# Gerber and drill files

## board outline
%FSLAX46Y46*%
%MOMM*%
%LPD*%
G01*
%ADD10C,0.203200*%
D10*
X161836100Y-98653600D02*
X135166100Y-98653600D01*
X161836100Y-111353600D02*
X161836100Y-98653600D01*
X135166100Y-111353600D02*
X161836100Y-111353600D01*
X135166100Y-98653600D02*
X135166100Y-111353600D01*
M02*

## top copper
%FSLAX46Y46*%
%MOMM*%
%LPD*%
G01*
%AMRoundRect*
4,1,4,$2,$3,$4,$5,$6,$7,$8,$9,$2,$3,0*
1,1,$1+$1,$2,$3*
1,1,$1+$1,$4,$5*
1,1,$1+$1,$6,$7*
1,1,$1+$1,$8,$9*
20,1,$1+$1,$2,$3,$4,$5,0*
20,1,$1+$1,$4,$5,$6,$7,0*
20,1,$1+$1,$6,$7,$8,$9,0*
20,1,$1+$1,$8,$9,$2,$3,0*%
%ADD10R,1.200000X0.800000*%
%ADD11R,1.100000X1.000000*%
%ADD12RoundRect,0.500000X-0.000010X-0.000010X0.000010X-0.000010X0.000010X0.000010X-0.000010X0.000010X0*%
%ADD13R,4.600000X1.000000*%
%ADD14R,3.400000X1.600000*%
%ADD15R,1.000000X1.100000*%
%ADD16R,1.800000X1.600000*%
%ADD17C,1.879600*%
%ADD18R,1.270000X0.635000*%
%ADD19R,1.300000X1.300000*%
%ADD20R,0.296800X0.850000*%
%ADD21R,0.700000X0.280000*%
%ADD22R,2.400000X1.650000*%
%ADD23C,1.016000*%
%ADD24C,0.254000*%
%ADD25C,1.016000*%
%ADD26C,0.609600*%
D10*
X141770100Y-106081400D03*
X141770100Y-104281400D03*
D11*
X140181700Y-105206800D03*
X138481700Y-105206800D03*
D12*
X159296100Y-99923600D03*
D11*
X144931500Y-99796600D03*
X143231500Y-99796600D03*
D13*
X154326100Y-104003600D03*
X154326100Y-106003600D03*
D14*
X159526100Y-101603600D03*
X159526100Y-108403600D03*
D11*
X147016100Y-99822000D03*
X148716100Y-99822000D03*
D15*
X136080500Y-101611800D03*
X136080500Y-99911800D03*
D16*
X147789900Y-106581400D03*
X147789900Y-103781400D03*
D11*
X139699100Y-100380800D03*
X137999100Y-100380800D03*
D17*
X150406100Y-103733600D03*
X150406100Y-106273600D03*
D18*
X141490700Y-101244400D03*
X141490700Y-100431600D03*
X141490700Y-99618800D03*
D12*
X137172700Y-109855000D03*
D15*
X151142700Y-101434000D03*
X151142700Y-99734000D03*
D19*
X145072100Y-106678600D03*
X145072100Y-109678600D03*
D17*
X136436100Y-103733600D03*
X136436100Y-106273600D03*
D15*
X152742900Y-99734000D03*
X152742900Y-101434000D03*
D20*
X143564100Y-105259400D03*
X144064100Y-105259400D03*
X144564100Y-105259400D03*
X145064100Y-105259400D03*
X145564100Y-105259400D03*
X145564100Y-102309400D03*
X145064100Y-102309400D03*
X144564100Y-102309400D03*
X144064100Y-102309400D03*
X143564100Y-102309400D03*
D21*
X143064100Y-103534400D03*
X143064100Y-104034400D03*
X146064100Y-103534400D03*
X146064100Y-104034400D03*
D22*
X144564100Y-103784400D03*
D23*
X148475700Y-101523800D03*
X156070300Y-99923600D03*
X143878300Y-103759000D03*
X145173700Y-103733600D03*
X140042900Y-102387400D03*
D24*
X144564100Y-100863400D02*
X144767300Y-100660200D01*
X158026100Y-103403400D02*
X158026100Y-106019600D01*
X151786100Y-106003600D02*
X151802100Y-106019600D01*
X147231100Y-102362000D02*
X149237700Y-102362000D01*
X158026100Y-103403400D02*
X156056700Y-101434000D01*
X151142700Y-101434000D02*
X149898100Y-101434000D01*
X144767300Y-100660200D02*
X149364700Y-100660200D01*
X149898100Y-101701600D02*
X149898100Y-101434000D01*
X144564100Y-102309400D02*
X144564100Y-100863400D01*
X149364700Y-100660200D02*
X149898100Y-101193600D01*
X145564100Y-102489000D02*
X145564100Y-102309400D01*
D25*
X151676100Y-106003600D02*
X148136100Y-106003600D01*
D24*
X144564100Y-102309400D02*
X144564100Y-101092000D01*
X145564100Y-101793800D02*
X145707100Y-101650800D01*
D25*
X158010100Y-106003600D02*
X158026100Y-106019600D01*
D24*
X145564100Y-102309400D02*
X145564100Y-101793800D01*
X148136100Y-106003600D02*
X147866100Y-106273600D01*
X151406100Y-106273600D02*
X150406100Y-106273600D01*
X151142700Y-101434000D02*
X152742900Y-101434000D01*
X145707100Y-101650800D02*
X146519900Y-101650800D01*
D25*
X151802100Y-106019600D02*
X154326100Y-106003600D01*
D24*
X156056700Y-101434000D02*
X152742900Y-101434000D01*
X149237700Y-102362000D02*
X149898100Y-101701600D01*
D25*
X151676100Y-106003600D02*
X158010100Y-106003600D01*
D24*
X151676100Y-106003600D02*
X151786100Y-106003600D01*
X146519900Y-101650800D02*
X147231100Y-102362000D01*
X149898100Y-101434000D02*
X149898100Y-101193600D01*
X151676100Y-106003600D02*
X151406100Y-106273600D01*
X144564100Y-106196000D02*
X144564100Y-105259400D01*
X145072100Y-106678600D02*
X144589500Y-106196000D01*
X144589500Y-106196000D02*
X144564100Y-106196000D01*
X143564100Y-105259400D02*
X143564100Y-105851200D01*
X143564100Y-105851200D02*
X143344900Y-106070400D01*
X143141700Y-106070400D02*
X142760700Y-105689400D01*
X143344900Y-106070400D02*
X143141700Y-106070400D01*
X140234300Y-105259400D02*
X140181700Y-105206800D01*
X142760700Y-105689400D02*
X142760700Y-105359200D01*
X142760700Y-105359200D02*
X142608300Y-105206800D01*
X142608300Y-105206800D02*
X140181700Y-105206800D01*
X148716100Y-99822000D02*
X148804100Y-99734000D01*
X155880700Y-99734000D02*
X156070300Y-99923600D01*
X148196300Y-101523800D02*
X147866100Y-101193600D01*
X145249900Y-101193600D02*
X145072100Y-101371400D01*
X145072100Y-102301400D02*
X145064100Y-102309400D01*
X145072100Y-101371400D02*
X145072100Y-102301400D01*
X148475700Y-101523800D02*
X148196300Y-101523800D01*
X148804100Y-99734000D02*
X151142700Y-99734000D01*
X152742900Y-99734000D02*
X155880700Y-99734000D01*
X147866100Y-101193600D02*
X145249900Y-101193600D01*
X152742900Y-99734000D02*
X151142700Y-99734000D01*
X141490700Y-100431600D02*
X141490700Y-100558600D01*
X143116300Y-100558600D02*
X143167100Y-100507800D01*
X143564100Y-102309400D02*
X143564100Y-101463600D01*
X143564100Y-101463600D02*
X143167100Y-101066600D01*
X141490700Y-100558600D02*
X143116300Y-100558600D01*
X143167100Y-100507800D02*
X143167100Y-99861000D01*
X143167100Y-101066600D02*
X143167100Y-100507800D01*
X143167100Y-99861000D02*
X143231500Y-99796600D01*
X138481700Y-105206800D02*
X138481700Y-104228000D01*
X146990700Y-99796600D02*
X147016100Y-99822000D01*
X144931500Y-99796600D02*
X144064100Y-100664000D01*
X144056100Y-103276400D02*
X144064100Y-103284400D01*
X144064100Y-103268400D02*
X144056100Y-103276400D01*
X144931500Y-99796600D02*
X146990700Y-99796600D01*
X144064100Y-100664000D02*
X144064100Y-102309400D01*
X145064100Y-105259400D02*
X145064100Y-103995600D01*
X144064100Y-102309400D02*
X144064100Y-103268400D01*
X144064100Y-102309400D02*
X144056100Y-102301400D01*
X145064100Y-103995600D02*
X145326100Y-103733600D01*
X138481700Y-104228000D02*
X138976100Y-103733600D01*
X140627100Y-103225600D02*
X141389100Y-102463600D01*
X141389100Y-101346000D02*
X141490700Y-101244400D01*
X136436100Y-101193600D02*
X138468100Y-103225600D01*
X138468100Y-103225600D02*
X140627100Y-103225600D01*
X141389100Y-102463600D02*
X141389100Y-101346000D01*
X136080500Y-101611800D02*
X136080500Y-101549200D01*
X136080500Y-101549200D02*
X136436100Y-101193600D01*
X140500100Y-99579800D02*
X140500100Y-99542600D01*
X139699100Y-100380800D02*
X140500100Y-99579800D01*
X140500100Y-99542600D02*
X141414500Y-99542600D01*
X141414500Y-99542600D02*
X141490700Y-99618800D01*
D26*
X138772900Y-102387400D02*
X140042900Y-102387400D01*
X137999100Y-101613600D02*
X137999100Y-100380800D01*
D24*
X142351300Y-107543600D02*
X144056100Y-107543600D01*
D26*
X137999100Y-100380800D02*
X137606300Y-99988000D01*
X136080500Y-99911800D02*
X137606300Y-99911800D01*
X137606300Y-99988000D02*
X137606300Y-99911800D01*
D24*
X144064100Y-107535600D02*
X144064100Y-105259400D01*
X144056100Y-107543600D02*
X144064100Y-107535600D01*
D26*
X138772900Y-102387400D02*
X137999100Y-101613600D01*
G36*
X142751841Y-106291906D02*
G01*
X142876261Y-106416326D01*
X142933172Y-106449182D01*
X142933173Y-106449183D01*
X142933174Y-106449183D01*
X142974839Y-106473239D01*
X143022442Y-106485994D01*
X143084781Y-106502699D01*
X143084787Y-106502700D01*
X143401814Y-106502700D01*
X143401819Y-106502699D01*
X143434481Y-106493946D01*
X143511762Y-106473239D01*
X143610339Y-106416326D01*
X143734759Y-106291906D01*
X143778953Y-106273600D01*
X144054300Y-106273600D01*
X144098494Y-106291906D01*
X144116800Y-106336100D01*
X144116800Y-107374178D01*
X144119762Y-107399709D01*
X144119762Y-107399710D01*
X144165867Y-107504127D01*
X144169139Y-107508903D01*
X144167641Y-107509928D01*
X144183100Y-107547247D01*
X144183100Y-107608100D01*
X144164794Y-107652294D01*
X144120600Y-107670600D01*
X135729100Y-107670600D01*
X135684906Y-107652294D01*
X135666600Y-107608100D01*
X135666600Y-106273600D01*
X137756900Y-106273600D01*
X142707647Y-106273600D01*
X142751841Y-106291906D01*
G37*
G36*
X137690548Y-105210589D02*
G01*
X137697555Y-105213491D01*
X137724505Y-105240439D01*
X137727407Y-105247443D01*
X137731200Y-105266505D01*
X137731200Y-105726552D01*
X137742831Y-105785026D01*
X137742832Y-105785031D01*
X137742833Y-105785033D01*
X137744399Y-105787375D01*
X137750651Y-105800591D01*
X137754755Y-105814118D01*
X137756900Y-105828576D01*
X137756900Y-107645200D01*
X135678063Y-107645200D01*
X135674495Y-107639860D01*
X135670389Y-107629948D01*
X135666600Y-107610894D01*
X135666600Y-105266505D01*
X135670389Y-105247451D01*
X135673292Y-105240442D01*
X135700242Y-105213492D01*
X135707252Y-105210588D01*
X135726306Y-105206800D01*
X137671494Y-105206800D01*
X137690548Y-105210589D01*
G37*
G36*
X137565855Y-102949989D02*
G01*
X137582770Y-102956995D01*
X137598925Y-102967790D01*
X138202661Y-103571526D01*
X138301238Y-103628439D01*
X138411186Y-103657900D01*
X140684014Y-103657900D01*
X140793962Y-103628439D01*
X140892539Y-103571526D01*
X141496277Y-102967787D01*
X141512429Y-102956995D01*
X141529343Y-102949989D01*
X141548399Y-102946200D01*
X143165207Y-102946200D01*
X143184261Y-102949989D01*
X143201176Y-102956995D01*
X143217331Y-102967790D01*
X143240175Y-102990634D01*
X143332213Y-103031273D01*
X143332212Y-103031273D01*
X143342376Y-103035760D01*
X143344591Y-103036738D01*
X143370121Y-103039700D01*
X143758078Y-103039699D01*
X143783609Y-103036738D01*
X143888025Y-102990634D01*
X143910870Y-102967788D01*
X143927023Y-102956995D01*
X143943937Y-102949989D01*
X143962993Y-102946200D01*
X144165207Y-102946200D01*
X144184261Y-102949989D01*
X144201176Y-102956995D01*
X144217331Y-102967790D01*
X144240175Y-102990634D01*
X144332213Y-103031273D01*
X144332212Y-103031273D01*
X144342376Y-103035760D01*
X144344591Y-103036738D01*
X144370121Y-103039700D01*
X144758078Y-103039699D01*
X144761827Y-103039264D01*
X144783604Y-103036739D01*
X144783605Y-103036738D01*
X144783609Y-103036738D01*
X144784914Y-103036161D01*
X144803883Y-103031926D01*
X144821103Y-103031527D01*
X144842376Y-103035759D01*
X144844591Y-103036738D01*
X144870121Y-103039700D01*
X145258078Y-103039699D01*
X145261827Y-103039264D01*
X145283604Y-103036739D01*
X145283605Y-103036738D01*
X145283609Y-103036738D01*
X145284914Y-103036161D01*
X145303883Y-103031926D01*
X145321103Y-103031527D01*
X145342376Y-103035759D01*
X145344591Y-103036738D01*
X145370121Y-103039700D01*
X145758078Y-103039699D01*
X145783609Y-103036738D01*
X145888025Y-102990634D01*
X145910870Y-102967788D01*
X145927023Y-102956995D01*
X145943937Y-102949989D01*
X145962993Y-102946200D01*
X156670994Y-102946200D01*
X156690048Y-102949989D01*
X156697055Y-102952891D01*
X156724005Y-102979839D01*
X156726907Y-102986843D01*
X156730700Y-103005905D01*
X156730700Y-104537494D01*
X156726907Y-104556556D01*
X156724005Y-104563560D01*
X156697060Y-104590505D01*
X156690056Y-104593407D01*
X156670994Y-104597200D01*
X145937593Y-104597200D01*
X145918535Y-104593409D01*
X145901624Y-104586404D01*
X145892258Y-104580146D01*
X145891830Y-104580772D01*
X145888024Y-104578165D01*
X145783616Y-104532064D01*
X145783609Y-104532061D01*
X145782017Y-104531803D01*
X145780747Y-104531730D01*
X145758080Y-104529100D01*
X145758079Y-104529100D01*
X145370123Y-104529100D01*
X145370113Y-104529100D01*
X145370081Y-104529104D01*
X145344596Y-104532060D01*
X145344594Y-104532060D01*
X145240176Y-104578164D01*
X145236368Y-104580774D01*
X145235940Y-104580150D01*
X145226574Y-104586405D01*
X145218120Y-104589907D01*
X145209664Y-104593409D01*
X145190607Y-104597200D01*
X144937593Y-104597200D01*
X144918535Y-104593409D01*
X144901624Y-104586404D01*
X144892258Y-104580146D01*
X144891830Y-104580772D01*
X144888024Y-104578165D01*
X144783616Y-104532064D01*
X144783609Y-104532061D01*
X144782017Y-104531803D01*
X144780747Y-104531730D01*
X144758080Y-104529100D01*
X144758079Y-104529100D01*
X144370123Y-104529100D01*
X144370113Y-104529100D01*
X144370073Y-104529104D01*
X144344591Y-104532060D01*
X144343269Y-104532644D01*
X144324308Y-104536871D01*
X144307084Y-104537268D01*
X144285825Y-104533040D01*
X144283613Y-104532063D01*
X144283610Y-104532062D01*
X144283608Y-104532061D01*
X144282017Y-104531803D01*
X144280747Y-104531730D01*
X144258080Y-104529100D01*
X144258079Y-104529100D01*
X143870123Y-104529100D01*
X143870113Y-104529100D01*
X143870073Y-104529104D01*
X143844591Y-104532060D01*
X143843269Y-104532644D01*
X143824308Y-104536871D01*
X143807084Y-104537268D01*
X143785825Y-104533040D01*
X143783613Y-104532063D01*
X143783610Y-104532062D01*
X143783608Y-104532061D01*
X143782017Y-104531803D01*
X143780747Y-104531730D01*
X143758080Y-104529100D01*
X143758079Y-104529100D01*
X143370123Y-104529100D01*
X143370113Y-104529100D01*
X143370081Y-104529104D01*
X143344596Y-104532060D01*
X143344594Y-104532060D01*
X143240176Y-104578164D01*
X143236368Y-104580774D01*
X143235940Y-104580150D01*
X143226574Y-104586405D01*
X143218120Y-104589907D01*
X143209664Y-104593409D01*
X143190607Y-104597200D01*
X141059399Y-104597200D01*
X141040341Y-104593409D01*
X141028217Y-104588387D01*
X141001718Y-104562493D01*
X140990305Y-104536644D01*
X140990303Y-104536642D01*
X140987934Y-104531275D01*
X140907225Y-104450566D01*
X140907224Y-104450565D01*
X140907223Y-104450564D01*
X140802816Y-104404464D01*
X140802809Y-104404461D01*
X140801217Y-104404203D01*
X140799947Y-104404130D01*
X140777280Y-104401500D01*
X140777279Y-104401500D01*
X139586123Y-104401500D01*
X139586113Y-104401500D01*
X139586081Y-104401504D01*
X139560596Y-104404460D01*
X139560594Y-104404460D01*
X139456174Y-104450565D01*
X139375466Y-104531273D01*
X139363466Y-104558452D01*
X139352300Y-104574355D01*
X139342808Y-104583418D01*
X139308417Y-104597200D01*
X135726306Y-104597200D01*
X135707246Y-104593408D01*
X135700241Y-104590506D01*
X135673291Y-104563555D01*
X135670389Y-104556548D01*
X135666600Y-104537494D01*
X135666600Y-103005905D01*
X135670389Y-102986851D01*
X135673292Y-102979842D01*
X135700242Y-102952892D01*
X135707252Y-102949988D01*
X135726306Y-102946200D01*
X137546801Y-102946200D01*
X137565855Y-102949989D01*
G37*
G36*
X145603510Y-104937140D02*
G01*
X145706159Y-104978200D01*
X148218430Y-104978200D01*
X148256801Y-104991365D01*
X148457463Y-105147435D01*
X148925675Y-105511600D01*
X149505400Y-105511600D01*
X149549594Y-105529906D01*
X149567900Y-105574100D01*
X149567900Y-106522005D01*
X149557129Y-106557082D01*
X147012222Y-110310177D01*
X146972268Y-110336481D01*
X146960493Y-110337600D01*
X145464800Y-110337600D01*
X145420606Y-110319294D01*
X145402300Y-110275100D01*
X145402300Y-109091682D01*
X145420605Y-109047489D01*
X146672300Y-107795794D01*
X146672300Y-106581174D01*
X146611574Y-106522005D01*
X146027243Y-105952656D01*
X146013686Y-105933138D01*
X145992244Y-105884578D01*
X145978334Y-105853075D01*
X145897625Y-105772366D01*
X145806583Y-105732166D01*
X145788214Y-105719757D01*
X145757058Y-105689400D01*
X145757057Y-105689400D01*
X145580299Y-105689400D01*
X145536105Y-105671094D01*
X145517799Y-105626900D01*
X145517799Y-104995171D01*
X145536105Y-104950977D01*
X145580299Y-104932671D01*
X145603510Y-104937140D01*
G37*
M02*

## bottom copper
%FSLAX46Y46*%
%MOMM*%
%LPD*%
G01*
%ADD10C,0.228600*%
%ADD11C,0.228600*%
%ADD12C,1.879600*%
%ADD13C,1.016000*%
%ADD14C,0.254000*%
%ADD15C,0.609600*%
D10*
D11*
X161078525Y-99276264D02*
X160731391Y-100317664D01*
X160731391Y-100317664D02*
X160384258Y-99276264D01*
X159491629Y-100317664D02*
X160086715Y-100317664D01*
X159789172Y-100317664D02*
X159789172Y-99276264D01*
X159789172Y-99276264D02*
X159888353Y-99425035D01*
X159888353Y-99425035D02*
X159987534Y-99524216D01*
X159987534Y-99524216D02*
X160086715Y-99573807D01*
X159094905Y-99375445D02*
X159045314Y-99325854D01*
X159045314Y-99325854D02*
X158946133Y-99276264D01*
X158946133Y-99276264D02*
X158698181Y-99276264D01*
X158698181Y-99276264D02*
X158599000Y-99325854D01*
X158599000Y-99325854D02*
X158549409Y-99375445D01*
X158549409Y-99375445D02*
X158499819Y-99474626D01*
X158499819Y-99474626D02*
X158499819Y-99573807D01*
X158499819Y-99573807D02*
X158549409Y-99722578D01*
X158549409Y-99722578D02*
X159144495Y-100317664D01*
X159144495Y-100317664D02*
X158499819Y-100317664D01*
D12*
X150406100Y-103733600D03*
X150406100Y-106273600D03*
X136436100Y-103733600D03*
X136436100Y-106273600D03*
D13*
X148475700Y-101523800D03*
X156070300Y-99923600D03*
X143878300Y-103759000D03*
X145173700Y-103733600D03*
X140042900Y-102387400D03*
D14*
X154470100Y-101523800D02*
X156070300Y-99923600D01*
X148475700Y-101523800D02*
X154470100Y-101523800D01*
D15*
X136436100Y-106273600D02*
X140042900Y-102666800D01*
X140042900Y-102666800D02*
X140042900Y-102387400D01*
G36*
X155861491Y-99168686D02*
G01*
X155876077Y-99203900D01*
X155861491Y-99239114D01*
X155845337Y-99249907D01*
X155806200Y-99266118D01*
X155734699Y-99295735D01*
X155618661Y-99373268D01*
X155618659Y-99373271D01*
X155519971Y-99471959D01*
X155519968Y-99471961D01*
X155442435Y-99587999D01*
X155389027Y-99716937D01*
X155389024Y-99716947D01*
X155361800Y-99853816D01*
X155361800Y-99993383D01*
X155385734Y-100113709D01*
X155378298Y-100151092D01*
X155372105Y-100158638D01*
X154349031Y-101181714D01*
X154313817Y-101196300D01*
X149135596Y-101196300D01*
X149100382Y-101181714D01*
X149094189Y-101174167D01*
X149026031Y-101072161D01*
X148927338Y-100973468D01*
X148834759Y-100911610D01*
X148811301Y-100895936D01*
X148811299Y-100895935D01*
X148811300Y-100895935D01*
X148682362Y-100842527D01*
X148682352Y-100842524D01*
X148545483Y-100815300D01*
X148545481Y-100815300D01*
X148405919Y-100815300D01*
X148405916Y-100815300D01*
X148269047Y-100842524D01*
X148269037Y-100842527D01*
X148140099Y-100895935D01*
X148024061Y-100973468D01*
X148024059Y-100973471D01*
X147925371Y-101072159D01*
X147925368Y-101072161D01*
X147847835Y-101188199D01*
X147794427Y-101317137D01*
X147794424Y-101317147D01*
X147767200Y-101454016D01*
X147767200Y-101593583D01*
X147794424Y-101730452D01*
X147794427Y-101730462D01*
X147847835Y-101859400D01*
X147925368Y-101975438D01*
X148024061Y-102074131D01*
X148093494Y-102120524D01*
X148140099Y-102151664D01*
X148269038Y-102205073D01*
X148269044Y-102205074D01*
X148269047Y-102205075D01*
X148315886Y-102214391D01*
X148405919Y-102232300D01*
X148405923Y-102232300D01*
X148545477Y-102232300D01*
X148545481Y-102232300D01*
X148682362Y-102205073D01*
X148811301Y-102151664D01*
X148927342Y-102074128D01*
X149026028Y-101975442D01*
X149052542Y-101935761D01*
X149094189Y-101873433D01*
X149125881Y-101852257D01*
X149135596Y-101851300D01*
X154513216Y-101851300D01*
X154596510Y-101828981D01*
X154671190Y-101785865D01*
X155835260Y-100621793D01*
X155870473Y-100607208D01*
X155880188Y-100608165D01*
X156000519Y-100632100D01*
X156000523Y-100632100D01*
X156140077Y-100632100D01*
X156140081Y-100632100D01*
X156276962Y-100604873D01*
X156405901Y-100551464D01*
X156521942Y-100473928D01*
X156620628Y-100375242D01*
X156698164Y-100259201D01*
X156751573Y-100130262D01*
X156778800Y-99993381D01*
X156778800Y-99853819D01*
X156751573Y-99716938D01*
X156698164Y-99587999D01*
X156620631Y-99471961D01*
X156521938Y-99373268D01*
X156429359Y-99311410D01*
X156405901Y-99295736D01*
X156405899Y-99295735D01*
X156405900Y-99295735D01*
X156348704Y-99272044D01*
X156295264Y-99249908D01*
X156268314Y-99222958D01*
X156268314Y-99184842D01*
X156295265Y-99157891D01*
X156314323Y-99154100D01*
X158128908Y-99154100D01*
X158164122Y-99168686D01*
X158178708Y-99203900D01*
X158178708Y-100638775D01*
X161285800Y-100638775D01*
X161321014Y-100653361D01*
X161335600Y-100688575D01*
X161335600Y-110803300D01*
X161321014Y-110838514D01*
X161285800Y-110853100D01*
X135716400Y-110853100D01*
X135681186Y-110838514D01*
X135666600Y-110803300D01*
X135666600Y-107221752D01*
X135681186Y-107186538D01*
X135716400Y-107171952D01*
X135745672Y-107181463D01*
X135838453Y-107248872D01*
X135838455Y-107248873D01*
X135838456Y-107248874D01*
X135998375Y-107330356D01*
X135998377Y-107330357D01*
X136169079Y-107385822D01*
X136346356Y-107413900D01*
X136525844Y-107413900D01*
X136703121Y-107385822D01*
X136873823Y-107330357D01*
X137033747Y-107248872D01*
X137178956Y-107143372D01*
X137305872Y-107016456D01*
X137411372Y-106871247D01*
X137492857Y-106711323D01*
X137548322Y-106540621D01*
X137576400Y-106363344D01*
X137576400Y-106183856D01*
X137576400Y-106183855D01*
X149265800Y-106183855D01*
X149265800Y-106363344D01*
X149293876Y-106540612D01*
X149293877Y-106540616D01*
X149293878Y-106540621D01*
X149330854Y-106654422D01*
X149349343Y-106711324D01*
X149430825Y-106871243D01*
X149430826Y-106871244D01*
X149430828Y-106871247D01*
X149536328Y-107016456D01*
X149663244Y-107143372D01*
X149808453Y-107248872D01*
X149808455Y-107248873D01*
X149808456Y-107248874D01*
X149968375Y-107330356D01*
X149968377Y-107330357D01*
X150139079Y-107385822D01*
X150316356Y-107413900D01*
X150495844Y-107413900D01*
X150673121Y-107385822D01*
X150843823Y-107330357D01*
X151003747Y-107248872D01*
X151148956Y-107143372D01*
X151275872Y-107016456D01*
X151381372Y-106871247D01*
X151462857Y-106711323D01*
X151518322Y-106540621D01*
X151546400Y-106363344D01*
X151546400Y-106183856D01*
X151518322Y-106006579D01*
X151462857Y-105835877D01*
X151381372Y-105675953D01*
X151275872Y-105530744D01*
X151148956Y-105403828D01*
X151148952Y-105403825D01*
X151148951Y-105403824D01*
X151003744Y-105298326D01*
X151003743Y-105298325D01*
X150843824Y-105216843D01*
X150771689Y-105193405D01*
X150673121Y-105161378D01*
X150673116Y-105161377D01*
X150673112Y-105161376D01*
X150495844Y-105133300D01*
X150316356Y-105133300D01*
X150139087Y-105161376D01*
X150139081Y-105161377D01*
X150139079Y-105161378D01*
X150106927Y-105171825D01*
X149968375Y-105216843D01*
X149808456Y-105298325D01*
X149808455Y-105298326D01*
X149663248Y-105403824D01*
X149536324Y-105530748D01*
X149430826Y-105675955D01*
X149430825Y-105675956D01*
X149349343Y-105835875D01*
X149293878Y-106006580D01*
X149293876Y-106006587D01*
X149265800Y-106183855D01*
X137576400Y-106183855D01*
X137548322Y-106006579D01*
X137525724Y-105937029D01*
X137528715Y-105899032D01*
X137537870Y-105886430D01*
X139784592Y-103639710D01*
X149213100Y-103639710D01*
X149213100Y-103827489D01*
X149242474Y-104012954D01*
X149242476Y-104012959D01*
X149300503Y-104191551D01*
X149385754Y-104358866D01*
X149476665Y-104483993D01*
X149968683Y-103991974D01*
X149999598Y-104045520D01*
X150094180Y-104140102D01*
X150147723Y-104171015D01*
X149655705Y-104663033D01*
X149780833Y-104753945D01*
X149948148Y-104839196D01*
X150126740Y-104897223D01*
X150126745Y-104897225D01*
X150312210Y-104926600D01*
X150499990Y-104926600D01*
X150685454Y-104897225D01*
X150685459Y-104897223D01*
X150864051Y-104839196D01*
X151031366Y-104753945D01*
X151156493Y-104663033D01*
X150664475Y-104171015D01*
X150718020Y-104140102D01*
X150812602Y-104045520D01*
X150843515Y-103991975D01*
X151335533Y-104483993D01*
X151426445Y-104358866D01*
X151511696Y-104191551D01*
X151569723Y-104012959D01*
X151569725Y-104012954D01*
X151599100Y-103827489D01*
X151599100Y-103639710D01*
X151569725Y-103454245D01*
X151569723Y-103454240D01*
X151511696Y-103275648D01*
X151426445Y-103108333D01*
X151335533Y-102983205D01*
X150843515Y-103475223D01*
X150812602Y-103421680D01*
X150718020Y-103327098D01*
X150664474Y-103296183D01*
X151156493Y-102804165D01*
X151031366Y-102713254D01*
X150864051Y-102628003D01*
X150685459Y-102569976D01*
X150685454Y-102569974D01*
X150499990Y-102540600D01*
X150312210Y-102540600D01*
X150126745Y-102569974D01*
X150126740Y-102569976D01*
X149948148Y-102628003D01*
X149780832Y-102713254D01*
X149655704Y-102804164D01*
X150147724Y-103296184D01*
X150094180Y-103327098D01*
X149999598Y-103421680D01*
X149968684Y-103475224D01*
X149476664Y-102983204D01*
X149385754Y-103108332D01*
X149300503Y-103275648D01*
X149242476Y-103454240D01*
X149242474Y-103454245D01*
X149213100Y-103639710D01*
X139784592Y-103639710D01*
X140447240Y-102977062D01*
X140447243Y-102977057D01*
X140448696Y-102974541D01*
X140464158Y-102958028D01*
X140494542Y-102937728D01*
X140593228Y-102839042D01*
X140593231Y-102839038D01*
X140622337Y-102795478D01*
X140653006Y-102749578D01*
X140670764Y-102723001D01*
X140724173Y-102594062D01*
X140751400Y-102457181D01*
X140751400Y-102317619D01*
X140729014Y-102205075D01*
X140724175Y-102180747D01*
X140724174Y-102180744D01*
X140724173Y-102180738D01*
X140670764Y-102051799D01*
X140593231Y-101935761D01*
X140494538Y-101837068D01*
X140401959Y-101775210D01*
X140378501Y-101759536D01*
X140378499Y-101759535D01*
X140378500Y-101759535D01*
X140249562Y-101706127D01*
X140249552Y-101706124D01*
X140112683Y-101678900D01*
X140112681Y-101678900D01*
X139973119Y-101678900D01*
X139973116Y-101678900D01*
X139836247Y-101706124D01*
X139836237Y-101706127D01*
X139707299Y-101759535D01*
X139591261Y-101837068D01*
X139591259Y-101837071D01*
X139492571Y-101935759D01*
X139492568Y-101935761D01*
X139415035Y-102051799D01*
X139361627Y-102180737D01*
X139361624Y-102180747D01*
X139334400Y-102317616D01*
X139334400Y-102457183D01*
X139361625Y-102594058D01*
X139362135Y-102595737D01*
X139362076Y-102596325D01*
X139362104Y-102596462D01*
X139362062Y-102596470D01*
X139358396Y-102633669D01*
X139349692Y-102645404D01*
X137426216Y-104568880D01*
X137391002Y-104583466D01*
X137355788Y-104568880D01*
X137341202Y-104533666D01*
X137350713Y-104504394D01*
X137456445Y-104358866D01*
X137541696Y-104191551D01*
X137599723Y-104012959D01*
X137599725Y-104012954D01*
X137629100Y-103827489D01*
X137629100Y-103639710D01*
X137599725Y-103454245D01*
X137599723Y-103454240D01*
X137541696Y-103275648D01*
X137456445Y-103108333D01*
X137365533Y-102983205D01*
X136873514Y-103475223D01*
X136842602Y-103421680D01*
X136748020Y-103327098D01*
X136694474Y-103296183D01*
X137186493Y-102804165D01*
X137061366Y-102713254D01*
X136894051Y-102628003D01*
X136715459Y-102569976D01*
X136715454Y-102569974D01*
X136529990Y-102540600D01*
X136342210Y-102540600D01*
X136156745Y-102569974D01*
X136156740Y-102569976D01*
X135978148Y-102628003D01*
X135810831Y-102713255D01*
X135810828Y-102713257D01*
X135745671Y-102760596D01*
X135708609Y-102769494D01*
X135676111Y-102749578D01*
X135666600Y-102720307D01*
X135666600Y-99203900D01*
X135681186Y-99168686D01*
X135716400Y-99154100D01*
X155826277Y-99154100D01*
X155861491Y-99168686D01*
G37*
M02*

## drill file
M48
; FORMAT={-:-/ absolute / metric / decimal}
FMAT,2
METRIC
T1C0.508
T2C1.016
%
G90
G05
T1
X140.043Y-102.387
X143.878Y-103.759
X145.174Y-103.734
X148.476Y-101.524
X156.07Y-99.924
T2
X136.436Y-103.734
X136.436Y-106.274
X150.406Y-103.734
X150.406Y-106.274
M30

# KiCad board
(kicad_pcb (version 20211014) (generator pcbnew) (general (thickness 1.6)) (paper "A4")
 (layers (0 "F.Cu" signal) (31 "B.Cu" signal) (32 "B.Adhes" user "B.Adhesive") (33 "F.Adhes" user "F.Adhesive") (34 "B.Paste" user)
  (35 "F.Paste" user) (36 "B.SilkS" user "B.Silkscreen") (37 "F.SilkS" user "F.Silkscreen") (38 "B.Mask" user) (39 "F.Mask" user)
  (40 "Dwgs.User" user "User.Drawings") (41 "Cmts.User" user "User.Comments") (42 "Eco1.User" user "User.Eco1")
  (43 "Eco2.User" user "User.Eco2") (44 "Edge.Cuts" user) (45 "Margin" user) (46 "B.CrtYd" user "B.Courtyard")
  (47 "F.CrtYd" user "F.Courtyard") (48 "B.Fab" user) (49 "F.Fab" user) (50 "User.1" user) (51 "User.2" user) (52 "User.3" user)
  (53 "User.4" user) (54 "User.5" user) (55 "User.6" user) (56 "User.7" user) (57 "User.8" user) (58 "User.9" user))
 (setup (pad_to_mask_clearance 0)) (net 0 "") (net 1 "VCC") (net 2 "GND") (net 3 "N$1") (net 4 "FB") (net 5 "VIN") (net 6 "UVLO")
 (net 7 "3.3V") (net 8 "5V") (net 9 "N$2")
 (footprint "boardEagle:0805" (layer "F.Cu") (at 141.7701 105.1814 90)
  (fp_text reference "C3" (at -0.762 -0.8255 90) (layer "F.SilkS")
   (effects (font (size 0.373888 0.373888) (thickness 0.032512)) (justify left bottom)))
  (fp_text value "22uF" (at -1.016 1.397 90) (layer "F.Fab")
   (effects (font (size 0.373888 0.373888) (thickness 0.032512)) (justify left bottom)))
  (pad "1" smd rect (at -0.9 0 90) (size 0.8 1.2) (layers "F.Cu" "F.Paste" "F.Mask") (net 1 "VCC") (solder_mask_margin 0.1016))
  (pad "2" smd rect (at 0.9 0 90) (size 0.8 1.2) (layers "F.Cu" "F.Paste" "F.Mask") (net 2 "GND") (solder_mask_margin 0.1016)))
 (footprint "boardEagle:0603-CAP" (layer "F.Cu") (at 139.3317 105.2068 180)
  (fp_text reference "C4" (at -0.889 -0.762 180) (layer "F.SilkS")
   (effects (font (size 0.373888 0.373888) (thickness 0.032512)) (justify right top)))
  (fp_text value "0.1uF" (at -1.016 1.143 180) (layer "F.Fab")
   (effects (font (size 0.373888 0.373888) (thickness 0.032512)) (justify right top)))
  (pad "1" smd rect (at -0.85 0 180) (size 1.1 1) (layers "F.Cu" "F.Paste" "F.Mask") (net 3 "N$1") (solder_mask_margin 0.1016))
  (pad "2" smd rect (at 0.85 0 180) (size 1.1 1) (layers "F.Cu" "F.Paste" "F.Mask") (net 2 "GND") (solder_mask_margin 0.1016)))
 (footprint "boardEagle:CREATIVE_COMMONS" (layer "F.Cu") (at 156.7561 120.2436)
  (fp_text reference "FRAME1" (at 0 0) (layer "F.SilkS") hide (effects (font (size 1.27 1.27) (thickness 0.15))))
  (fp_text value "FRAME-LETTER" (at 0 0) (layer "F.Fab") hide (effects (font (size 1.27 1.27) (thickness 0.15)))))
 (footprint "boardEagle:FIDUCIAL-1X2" (layer "F.Cu") (at 159.2961 99.9236)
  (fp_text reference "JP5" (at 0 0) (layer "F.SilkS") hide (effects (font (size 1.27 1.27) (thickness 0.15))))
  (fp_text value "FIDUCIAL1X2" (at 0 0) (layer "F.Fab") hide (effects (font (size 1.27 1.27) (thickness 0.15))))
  (pad "1" smd roundrect (at 0 0) (size 1 1) (layers "F.Cu" "F.Mask") (roundrect_rratio 0.5) (solder_mask_margin 0.1016)))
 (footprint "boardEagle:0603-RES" (layer "F.Cu") (at 144.0815 99.7966 180)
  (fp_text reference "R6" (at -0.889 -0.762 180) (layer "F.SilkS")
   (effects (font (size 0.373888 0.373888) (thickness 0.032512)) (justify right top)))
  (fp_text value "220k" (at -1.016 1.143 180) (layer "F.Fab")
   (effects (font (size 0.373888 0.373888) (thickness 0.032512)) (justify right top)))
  (pad "1" smd rect (at -0.85 0 180) (size 1.1 1) (layers "F.Cu" "F.Paste" "F.Mask") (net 2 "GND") (solder_mask_margin 0.1016))
  (pad "2" smd rect (at 0.85 0 180) (size 1.1 1) (layers "F.Cu" "F.Paste" "F.Mask") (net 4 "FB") (solder_mask_margin 0.1016)))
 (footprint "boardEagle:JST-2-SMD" (layer "F.Cu") (at 158.0261 105.0036 -90)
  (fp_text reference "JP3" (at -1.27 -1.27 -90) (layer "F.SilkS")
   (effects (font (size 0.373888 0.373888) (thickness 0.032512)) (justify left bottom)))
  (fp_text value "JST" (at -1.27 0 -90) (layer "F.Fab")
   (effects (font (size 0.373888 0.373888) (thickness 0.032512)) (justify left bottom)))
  (pad "1" smd rect (at -1 3.7 270) (size 1 4.6) (layers "F.Cu" "F.Paste" "F.Mask") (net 2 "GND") (solder_mask_margin 0.1016))
  (pad "2" smd rect (at 1 3.7 270) (size 1 4.6) (layers "F.Cu" "F.Paste" "F.Mask") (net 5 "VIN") (solder_mask_margin 0.1016))
  (pad "NC1" smd rect (at -3.4 -1.5) (size 3.4 1.6) (layers "F.Cu" "F.Paste" "F.Mask") (solder_mask_margin 0.1016))
  (pad "NC2" smd rect (at 3.4 -1.5) (size 3.4 1.6) (layers "F.Cu" "F.Paste" "F.Mask") (solder_mask_margin 0.1016)))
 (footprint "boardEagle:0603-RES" (layer "F.Cu") (at 147.8661 99.822)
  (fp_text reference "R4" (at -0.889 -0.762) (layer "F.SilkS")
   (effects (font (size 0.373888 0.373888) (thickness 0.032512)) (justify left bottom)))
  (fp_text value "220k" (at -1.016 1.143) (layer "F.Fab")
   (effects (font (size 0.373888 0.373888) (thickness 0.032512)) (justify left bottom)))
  (pad "1" smd rect (at -0.85 0) (size 1.1 1) (layers "F.Cu" "F.Paste" "F.Mask") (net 2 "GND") (solder_mask_margin 0.1016))
  (pad "2" smd rect (at 0.85 0) (size 1.1 1) (layers "F.Cu" "F.Paste" "F.Mask") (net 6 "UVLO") (solder_mask_margin 0.1016)))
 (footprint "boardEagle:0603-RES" (layer "F.Cu") (at 136.0805 100.7618 90)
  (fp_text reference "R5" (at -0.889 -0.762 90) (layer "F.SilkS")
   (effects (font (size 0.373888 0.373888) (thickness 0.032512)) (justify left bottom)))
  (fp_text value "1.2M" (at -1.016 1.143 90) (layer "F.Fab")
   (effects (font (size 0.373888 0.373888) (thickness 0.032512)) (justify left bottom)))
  (pad "1" smd rect (at -0.85 0 90) (size 1.1 1) (layers "F.Cu" "F.Paste" "F.Mask") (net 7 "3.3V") (solder_mask_margin 0.1016))
  (pad "2" smd rect (at 0.85 0 90) (size 1.1 1) (layers "F.Cu" "F.Paste" "F.Mask") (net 1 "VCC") (solder_mask_margin 0.1016)))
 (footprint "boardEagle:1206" (layer "F.Cu") (at 147.7899 105.1814 90)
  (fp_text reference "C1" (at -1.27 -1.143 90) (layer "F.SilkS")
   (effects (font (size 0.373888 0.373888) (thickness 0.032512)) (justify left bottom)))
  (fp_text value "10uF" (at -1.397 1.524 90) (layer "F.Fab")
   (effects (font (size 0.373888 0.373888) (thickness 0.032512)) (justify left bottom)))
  (pad "1" smd rect (at -1.4 0 90) (size 1.6 1.8) (layers "F.Cu" "F.Paste" "F.Mask") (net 5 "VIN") (solder_mask_margin 0.1016))
  (pad "2" smd rect (at 1.4 0 90) (size 1.6 1.8) (layers "F.Cu" "F.Paste" "F.Mask") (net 2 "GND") (solder_mask_margin 0.1016)))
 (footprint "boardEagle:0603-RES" (layer "F.Cu") (at 138.8491 100.3808 180)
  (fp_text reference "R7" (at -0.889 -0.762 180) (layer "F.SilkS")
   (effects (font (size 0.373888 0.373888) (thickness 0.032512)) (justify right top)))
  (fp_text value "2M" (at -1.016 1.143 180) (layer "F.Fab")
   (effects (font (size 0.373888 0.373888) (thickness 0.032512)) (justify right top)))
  (pad "1" smd rect (at -0.85 0 180) (size 1.1 1) (layers "F.Cu" "F.Paste" "F.Mask") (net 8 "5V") (solder_mask_margin 0.1016))
  (pad "2" smd rect (at 0.85 0 180) (size 1.1 1) (layers "F.Cu" "F.Paste" "F.Mask") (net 1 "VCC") (solder_mask_margin 0.1016)))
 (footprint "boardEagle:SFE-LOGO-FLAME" (layer "F.Cu") (at 138.8745 110.5662)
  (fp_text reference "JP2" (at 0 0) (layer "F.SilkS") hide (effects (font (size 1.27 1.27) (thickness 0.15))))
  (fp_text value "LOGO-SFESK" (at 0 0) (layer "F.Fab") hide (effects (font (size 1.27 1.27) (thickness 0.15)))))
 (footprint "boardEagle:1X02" (layer "F.Cu") (at 150.4061 103.7336 -90)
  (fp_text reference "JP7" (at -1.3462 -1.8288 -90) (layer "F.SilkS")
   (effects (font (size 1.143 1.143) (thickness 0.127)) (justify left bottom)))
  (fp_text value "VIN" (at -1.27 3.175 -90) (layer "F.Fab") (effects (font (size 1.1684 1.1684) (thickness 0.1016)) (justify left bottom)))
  (pad "1" thru_hole circle (at 0 0) (size 1.8796 1.8796) (drill 1.016) (layers *.Cu *.Mask) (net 2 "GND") (solder_mask_margin 0.1016))
  (pad "2" thru_hole circle (at 2.54 0) (size 1.8796 1.8796) (drill 1.016) (layers *.Cu *.Mask) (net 5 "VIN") (solder_mask_margin 0.1016)))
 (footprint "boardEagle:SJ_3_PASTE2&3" (layer "F.Cu") (at 141.4907 100.4316 90)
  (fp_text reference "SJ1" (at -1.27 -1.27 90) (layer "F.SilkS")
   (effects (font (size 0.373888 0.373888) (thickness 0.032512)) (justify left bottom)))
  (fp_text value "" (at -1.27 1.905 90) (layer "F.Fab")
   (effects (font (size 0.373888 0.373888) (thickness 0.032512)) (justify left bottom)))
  (pad "1" smd rect (at -0.8128 0 90) (size 0.635 1.27) (layers "F.Cu" "F.Mask") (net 7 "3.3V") (solder_mask_margin 0.1016))
  (pad "2" smd rect (at 0 0 90) (size 0.635 1.27) (layers "F.Cu" "F.Mask") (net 4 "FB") (solder_mask_margin 0.1016))
  (pad "3" smd rect (at 0.8128 0 90) (size 0.635 1.27) (layers "F.Cu" "F.Mask") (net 8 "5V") (solder_mask_margin 0.1016)))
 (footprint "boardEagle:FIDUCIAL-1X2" (layer "F.Cu") (at 137.1727 109.855)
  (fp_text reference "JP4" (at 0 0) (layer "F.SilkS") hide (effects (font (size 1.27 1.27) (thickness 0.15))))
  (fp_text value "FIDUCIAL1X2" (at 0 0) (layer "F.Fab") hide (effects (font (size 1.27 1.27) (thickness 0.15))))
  (pad "1" smd roundrect (at 0 0) (size 1 1) (layers "F.Cu" "F.Mask") (roundrect_rratio 0.5) (solder_mask_margin 0.1016)))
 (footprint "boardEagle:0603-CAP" (layer "F.Cu") (at 151.1427 100.584 90)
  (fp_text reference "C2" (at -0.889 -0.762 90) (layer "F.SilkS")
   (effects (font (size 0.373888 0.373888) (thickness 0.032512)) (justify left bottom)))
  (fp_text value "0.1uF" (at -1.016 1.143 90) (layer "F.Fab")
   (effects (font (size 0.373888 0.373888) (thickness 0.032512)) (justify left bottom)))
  (pad "1" smd rect (at -0.85 0 90) (size 1.1 1) (layers "F.Cu" "F.Paste" "F.Mask") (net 5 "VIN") (solder_mask_margin 0.1016))
  (pad "2" smd rect (at 0.85 0 90) (size 1.1 1) (layers "F.Cu" "F.Paste" "F.Mask") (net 6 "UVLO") (solder_mask_margin 0.1016)))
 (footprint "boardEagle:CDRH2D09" (layer "F.Cu") (at 145.0721 108.1786 -90)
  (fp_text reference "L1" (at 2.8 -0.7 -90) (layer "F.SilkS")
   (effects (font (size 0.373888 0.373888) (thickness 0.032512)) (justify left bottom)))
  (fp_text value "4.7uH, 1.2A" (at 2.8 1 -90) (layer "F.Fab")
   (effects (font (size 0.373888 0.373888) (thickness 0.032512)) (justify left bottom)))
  (pad "P$1" smd rect (at -1.5 0) (size 1.3 1.3) (layers "F.Cu" "F.Paste" "F.Mask") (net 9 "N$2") (solder_mask_margin 0.1016))
  (pad "P$2" smd rect (at 1.5 0) (size 1.3 1.3) (layers "F.Cu" "F.Paste" "F.Mask") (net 5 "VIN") (solder_mask_margin 0.1016)))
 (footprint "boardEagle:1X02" (layer "F.Cu") (at 136.4361 103.7336 -90)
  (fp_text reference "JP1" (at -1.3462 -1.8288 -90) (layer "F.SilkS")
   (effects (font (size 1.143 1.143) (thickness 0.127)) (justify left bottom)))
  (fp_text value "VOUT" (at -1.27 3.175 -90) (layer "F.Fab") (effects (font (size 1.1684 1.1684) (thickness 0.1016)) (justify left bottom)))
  (pad "1" thru_hole circle (at 0 0) (size 1.8796 1.8796) (drill 1.016) (layers *.Cu *.Mask) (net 2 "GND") (solder_mask_margin 0.1016))
  (pad "2" thru_hole circle (at 2.54 0) (size 1.8796 1.8796) (drill 1.016) (layers *.Cu *.Mask) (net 1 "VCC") (solder_mask_margin 0.1016)))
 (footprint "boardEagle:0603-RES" (layer "F.Cu") (at 152.7429 100.584 -90)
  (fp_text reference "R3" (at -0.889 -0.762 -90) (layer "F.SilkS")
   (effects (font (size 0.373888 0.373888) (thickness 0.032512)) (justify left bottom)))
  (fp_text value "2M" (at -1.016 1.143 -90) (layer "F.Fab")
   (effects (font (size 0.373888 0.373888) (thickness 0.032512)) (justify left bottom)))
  (pad "1" smd rect (at -0.85 0 270) (size 1.1 1) (layers "F.Cu" "F.Paste" "F.Mask") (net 6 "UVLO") (solder_mask_margin 0.1016))
  (pad "2" smd rect (at 0.85 0 270) (size 1.1 1) (layers "F.Cu" "F.Paste" "F.Mask") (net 5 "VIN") (solder_mask_margin 0.1016)))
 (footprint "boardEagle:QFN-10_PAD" (layer "F.Cu") (at 144.5641 103.7844)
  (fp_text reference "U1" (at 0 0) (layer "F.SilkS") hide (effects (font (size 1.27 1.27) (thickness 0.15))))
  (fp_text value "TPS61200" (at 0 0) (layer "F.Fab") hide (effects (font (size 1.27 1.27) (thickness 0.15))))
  (pad "1" smd rect (at -1 1.475 90) (size 0.85 0.2968) (layers "F.Cu" "F.Paste" "F.Mask") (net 3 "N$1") (solder_mask_margin 0.1016))
  (pad "2" smd rect (at -0.5 1.475 90) (size 0.85 0.2968) (layers "F.Cu" "F.Paste" "F.Mask") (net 1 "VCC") (solder_mask_margin 0.1016))
  (pad "3" smd rect (at 0 1.475 90) (size 0.85 0.2968) (layers "F.Cu" "F.Paste" "F.Mask") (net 9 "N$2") (solder_mask_margin 0.1016))
  (pad "4" smd rect (at 0.5 1.475 90) (size 0.85 0.2968) (layers "F.Cu" "F.Paste" "F.Mask") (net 2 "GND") (solder_mask_margin 0.1016))
  (pad "5" smd rect (at 1 1.475 90) (size 0.85 0.2968) (layers "F.Cu" "F.Paste" "F.Mask") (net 5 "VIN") (solder_mask_margin 0.1016))
  (pad "6" smd rect (at 1 -1.475 90) (size 0.85 0.2968) (layers "F.Cu" "F.Paste" "F.Mask") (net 5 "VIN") (solder_mask_margin 0.1016))
  (pad "7" smd rect (at 0.5 -1.475 90) (size 0.85 0.2968) (layers "F.Cu" "F.Paste" "F.Mask") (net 6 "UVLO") (solder_mask_margin 0.1016))
  (pad "8" smd rect (at 0 -1.475 90) (size 0.85 0.2968) (layers "F.Cu" "F.Paste" "F.Mask") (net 5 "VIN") (solder_mask_margin 0.1016))
  (pad "9" smd rect (at -0.5 -1.475 90) (size 0.85 0.2968) (layers "F.Cu" "F.Paste" "F.Mask") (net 2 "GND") (solder_mask_margin 0.1016))
  (pad "10" smd rect (at -1 -1.475 90) (size 0.85 0.2968) (layers "F.Cu" "F.Paste" "F.Mask") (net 4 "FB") (solder_mask_margin 0.1016))
  (pad "11" smd rect (at -1.5 -0.25 180) (size 0.7 0.28) (layers "F.Cu" "F.Paste" "F.Mask") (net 2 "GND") (solder_mask_margin 0.1016))
  (pad "12" smd rect (at -1.5 0.25 180) (size 0.7 0.28) (layers "F.Cu" "F.Paste" "F.Mask") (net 2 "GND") (solder_mask_margin 0.1016))
  (pad "13" smd rect (at 1.5 -0.25 180) (size 0.7 0.28) (layers "F.Cu" "F.Paste" "F.Mask") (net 2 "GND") (solder_mask_margin 0.1016))
  (pad "14" smd rect (at 1.5 0.25 180) (size 0.7 0.28) (layers "F.Cu" "F.Paste" "F.Mask") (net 2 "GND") (solder_mask_margin 0.1016))
  (pad "15" smd rect (at 0 0 90) (size 1.65 2.4) (layers "F.Cu" "F.Mask") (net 2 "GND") (solder_mask_margin 0.1016)))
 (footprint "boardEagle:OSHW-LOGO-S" (layer "B.Cu") (at 159.9311 109.7026 180)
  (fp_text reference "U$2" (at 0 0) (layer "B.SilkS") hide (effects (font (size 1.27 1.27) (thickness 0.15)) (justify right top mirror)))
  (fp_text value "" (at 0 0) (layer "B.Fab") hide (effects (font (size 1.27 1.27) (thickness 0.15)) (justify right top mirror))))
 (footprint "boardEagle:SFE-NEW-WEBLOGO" (layer "B.Cu") (at 154.5268 111.1442 180)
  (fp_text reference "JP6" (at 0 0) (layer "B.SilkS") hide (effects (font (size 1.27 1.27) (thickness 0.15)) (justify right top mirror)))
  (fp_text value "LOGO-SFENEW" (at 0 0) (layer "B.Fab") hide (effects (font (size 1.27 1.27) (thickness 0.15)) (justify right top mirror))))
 (gr_line (start 161.8361 98.6536) (end 135.1661 98.6536) (layer "Edge.Cuts") (width 0.2032))
 (gr_line (start 161.8361 111.3536) (end 161.8361 98.6536) (layer "Edge.Cuts") (width 0.2032))
 (gr_line (start 135.1661 111.3536) (end 161.8361 111.3536) (layer "Edge.Cuts") (width 0.2032))
 (gr_line (start 135.1661 98.6536) (end 135.1661 111.3536) (layer "Edge.Cuts") (width 0.2032))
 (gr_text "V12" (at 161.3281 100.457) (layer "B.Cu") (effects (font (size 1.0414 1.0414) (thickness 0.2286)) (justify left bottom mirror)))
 (segment (start 144.5641 100.8634) (end 144.7673 100.6602) (width 0.254) (layer "F.Cu") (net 5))
 (segment (start 158.0261 103.4034) (end 158.0261 106.0196) (width 0.254) (layer "F.Cu") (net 5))
 (segment (start 151.7861 106.0036) (end 151.8021 106.0196) (width 0.254) (layer "F.Cu") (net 5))
 (segment (start 147.2311 102.362) (end 149.2377 102.362) (width 0.254) (layer "F.Cu") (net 5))
 (segment (start 158.0261 103.4034) (end 156.0567 101.434) (width 0.254) (layer "F.Cu") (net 5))
 (segment (start 151.1427 101.434) (end 149.8981 101.434) (width 0.254) (layer "F.Cu") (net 5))
 (segment (start 144.7673 100.6602) (end 149.3647 100.6602) (width 0.254) (layer "F.Cu") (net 5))
 (segment (start 149.8981 101.7016) (end 149.8981 101.434) (width 0.254) (layer "F.Cu") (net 5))
 (segment (start 144.5641 102.3094) (end 144.5641 100.8634) (width 0.254) (layer "F.Cu") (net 5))
 (segment (start 149.3647 100.6602) (end 149.8981 101.1936) (width 0.254) (layer "F.Cu") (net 5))
 (segment (start 145.5641 102.489) (end 145.5641 102.3094) (width 0.254) (layer "F.Cu") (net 5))
 (segment (start 151.6761 106.0036) (end 148.1361 106.0036) (width 1.016) (layer "F.Cu") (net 5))
 (segment (start 144.5641 102.3094) (end 144.5641 101.092) (width 0.254) (layer "F.Cu") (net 5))
 (segment (start 145.5641 101.7938) (end 145.7071 101.6508) (width 0.254) (layer "F.Cu") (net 5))
 (segment (start 158.0101 106.0036) (end 158.0261 106.0196) (width 1.016) (layer "F.Cu") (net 5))
 (segment (start 145.5641 102.3094) (end 145.5641 101.7938) (width 0.254) (layer "F.Cu") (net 5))
 (segment (start 148.1361 106.0036) (end 147.8661 106.2736) (width 0.254) (layer "F.Cu") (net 5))
 (segment (start 151.4061 106.2736) (end 150.4061 106.2736) (width 0.254) (layer "F.Cu") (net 5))
 (segment (start 151.1427 101.434) (end 152.7429 101.434) (width 0.254) (layer "F.Cu") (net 5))
 (segment (start 145.7071 101.6508) (end 146.5199 101.6508) (width 0.254) (layer "F.Cu") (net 5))
 (segment (start 151.8021 106.0196) (end 154.3261 106.0036) (width 1.016) (layer "F.Cu") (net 5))
 (segment (start 156.0567 101.434) (end 152.7429 101.434) (width 0.254) (layer "F.Cu") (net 5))
 (segment (start 149.2377 102.362) (end 149.8981 101.7016) (width 0.254) (layer "F.Cu") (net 5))
 (segment (start 151.6761 106.0036) (end 158.0101 106.0036) (width 1.016) (layer "F.Cu") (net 5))
 (segment (start 151.6761 106.0036) (end 151.7861 106.0036) (width 0.254) (layer "F.Cu") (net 5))
 (segment (start 146.5199 101.6508) (end 147.2311 102.362) (width 0.254) (layer "F.Cu") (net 5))
 (segment (start 149.8981 101.434) (end 149.8981 101.1936) (width 0.254) (layer "F.Cu") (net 5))
 (segment (start 151.6761 106.0036) (end 151.4061 106.2736) (width 0.254) (layer "F.Cu") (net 5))
 (segment (start 144.5641 106.196) (end 144.5641 105.2594) (width 0.254) (layer "F.Cu") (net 9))
 (segment (start 145.0721 106.6786) (end 144.5895 106.196) (width 0.254) (layer "F.Cu") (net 9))
 (segment (start 144.5895 106.196) (end 144.5641 106.196) (width 0.254) (layer "F.Cu") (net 9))
 (segment (start 143.5641 105.2594) (end 143.5641 105.8512) (width 0.254) (layer "F.Cu") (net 3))
 (segment (start 143.5641 105.8512) (end 143.3449 106.0704) (width 0.254) (layer "F.Cu") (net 3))
 (segment (start 143.1417 106.0704) (end 142.7607 105.6894) (width 0.254) (layer "F.Cu") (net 3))
 (segment (start 143.3449 106.0704) (end 143.1417 106.0704) (width 0.254) (layer "F.Cu") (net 3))
 (segment (start 140.2343 105.2594) (end 140.1817 105.2068) (width 0.254) (layer "F.Cu") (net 3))
 (segment (start 142.7607 105.6894) (end 142.7607 105.3592) (width 0.254) (layer "F.Cu") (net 3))
 (segment (start 142.7607 105.3592) (end 142.6083 105.2068) (width 0.254) (layer "F.Cu") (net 3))
 (segment (start 142.6083 105.2068) (end 140.1817 105.2068) (width 0.254) (layer "F.Cu") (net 3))
 (segment (start 148.7161 99.822) (end 148.8041 99.734) (width 0.254) (layer "F.Cu") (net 6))
 (segment (start 155.8807 99.734) (end 156.0703 99.9236) (width 0.254) (layer "F.Cu") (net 6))
 (segment (start 148.1963 101.5238) (end 147.8661 101.1936) (width 0.254) (layer "F.Cu") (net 6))
 (segment (start 145.2499 101.1936) (end 145.0721 101.3714) (width 0.254) (layer "F.Cu") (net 6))
 (segment (start 145.0721 102.3014) (end 145.0641 102.3094) (width 0.254) (layer "F.Cu") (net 6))
 (segment (start 145.0721 101.3714) (end 145.0721 102.3014) (width 0.254) (layer "F.Cu") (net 6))
 (segment (start 148.4757 101.5238) (end 148.1963 101.5238) (width 0.254) (layer "F.Cu") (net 6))
 (segment (start 148.8041 99.734) (end 151.1427 99.734) (width 0.254) (layer "F.Cu") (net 6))
 (segment (start 152.7429 99.734) (end 155.8807 99.734) (width 0.254) (layer "F.Cu") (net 6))
 (segment (start 147.8661 101.1936) (end 145.2499 101.1936) (width 0.254) (layer "F.Cu") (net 6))
 (segment (start 152.7429 99.734) (end 151.1427 99.734) (width 0.254) (layer "F.Cu") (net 6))
 (via (at 148.4757 101.5238) (size 1.016) (drill 0.508) (layers "F.Cu" "B.Cu") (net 6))
 (via (at 156.0703 99.9236) (size 1.016) (drill 0.508) (layers "F.Cu" "B.Cu") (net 6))
 (segment (start 154.4701 101.5238) (end 156.0703 99.9236) (width 0.254) (layer "B.Cu") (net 6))
 (segment (start 148.4757 101.5238) (end 154.4701 101.5238) (width 0.254) (layer "B.Cu") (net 6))
 (segment (start 141.4907 100.4316) (end 141.4907 100.5586) (width 0.254) (layer "F.Cu") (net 4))
 (segment (start 143.1163 100.5586) (end 143.1671 100.5078) (width 0.254) (layer "F.Cu") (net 4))
 (segment (start 143.5641 102.3094) (end 143.5641 101.4636) (width 0.254) (layer "F.Cu") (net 4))
 (segment (start 143.5641 101.4636) (end 143.1671 101.0666) (width 0.254) (layer "F.Cu") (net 4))
 (segment (start 141.4907 100.5586) (end 143.1163 100.5586) (width 0.254) (layer "F.Cu") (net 4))
 (segment (start 143.1671 100.5078) (end 143.1671 99.861) (width 0.254) (layer "F.Cu") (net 4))
 (segment (start 143.1671 101.0666) (end 143.1671 100.5078) (width 0.254) (layer "F.Cu") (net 4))
 (segment (start 143.1671 99.861) (end 143.2315 99.7966) (width 0.254) (layer "F.Cu") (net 4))
 (segment (start 138.4817 105.2068) (end 138.4817 104.228) (width 0.254) (layer "F.Cu") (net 2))
 (segment (start 146.9907 99.7966) (end 147.0161 99.822) (width 0.254) (layer "F.Cu") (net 2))
 (segment (start 144.9315 99.7966) (end 144.0641 100.664) (width 0.254) (layer "F.Cu") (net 2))
 (segment (start 144.0561 103.2764) (end 144.0641 103.2844) (width 0.254) (layer "F.Cu") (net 2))
 (segment (start 144.0641 103.2684) (end 144.0561 103.2764) (width 0.254) (layer "F.Cu") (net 2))
 (segment (start 144.9315 99.7966) (end 146.9907 99.7966) (width 0.254) (layer "F.Cu") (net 2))
 (segment (start 144.0641 100.664) (end 144.0641 102.3094) (width 0.254) (layer "F.Cu") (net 2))
 (segment (start 145.0641 105.2594) (end 145.0641 103.9956) (width 0.254) (layer "F.Cu") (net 2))
 (segment (start 144.0641 102.3094) (end 144.0641 103.2684) (width 0.254) (layer "F.Cu") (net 2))
 (segment (start 144.0641 102.3094) (end 144.0561 102.3014) (width 0.254) (layer "F.Cu") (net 2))
 (segment (start 145.0641 103.9956) (end 145.3261 103.7336) (width 0.254) (layer "F.Cu") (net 2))
 (segment (start 138.4817 104.228) (end 138.9761 103.7336) (width 0.254) (layer "F.Cu") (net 2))
 (via (at 143.8783 103.759) (size 1.016) (drill 0.508) (layers "F.Cu" "B.Cu") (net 2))
 (via (at 145.1737 103.7336) (size 1.016) (drill 0.508) (layers "F.Cu" "B.Cu") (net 2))
 (segment (start 140.6271 103.2256) (end 141.3891 102.4636) (width 0.254) (layer "F.Cu") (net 7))
 (segment (start 141.3891 101.346) (end 141.4907 101.2444) (width 0.254) (layer "F.Cu") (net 7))
 (segment (start 136.4361 101.1936) (end 138.4681 103.2256) (width 0.254) (layer "F.Cu") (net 7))
 (segment (start 138.4681 103.2256) (end 140.6271 103.2256) (width 0.254) (layer "F.Cu") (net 7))
 (segment (start 141.3891 102.4636) (end 141.3891 101.346) (width 0.254) (layer "F.Cu") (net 7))
 (segment (start 136.0805 101.6118) (end 136.0805 101.5492) (width 0.254) (layer "F.Cu") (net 7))
 (segment (start 136.0805 101.5492) (end 136.4361 101.1936) (width 0.254) (layer "F.Cu") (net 7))
 (segment (start 140.5001 99.5798) (end 140.5001 99.5426) (width 0.254) (layer "F.Cu") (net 8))
 (segment (start 139.6991 100.3808) (end 140.5001 99.5798) (width 0.254) (layer "F.Cu") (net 8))
 (segment (start 140.5001 99.5426) (end 141.4145 99.5426) (width 0.254) (layer "F.Cu") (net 8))
 (segment (start 141.4145 99.5426) (end 141.4907 99.6188) (width 0.254) (layer "F.Cu") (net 8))
 (segment (start 138.7729 102.3874) (end 140.0429 102.3874) (width 0.6096) (layer "F.Cu") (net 1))
 (segment (start 137.9991 101.6136) (end 137.9991 100.3808) (width 0.6096) (layer "F.Cu") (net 1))
 (segment (start 142.3513 107.5436) (end 144.0561 107.5436) (width 0.254) (layer "F.Cu") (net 1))
 (segment (start 137.9991 100.3808) (end 137.6063 99.988) (width 0.6096) (layer "F.Cu") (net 1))
 (segment (start 136.0805 99.9118) (end 137.6063 99.9118) (width 0.6096) (layer "F.Cu") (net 1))
 (segment (start 137.6063 99.988) (end 137.6063 99.9118) (width 0.6096) (layer "F.Cu") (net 1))
 (segment (start 144.0641 107.5356) (end 144.0641 105.2594) (width 0.254) (layer "F.Cu") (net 1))
 (segment (start 144.0561 107.5436) (end 144.0641 107.5356) (width 0.254) (layer "F.Cu") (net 1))
 (segment (start 138.7729 102.3874) (end 137.9991 101.6136) (width 0.6096) (layer "F.Cu") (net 1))
 (via (at 140.0429 102.3874) (size 1.016) (drill 0.508) (layers "F.Cu" "B.Cu") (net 1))
 (segment (start 136.4361 106.2736) (end 140.0429 102.6668) (width 0.6096) (layer "B.Cu") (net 1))
 (segment (start 140.0429 102.6668) (end 140.0429 102.3874) (width 0.6096) (layer "B.Cu") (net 1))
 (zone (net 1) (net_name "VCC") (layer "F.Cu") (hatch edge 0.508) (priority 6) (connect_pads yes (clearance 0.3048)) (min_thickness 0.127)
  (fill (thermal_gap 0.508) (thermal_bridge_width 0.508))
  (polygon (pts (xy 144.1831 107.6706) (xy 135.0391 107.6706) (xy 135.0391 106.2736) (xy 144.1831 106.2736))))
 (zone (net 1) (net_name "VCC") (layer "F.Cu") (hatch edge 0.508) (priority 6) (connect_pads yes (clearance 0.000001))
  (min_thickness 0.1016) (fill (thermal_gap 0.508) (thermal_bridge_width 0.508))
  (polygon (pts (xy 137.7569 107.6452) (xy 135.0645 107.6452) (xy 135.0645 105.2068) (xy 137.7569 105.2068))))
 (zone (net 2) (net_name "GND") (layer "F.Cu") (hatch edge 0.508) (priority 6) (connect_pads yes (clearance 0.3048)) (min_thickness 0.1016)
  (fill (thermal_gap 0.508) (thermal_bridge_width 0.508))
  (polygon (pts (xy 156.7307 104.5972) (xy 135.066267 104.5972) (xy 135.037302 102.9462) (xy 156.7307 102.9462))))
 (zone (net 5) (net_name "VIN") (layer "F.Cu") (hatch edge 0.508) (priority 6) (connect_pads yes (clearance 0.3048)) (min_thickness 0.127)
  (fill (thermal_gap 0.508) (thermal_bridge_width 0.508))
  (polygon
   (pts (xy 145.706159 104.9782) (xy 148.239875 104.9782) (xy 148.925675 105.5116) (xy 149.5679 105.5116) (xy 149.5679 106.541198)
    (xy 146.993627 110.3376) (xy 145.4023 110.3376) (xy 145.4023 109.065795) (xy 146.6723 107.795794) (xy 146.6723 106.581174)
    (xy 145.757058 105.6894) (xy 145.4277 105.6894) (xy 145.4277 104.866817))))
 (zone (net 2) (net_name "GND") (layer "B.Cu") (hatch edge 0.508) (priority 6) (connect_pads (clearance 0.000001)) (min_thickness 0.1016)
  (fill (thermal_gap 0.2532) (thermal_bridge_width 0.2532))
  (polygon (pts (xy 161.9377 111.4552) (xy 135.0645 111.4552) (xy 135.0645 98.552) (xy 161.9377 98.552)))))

